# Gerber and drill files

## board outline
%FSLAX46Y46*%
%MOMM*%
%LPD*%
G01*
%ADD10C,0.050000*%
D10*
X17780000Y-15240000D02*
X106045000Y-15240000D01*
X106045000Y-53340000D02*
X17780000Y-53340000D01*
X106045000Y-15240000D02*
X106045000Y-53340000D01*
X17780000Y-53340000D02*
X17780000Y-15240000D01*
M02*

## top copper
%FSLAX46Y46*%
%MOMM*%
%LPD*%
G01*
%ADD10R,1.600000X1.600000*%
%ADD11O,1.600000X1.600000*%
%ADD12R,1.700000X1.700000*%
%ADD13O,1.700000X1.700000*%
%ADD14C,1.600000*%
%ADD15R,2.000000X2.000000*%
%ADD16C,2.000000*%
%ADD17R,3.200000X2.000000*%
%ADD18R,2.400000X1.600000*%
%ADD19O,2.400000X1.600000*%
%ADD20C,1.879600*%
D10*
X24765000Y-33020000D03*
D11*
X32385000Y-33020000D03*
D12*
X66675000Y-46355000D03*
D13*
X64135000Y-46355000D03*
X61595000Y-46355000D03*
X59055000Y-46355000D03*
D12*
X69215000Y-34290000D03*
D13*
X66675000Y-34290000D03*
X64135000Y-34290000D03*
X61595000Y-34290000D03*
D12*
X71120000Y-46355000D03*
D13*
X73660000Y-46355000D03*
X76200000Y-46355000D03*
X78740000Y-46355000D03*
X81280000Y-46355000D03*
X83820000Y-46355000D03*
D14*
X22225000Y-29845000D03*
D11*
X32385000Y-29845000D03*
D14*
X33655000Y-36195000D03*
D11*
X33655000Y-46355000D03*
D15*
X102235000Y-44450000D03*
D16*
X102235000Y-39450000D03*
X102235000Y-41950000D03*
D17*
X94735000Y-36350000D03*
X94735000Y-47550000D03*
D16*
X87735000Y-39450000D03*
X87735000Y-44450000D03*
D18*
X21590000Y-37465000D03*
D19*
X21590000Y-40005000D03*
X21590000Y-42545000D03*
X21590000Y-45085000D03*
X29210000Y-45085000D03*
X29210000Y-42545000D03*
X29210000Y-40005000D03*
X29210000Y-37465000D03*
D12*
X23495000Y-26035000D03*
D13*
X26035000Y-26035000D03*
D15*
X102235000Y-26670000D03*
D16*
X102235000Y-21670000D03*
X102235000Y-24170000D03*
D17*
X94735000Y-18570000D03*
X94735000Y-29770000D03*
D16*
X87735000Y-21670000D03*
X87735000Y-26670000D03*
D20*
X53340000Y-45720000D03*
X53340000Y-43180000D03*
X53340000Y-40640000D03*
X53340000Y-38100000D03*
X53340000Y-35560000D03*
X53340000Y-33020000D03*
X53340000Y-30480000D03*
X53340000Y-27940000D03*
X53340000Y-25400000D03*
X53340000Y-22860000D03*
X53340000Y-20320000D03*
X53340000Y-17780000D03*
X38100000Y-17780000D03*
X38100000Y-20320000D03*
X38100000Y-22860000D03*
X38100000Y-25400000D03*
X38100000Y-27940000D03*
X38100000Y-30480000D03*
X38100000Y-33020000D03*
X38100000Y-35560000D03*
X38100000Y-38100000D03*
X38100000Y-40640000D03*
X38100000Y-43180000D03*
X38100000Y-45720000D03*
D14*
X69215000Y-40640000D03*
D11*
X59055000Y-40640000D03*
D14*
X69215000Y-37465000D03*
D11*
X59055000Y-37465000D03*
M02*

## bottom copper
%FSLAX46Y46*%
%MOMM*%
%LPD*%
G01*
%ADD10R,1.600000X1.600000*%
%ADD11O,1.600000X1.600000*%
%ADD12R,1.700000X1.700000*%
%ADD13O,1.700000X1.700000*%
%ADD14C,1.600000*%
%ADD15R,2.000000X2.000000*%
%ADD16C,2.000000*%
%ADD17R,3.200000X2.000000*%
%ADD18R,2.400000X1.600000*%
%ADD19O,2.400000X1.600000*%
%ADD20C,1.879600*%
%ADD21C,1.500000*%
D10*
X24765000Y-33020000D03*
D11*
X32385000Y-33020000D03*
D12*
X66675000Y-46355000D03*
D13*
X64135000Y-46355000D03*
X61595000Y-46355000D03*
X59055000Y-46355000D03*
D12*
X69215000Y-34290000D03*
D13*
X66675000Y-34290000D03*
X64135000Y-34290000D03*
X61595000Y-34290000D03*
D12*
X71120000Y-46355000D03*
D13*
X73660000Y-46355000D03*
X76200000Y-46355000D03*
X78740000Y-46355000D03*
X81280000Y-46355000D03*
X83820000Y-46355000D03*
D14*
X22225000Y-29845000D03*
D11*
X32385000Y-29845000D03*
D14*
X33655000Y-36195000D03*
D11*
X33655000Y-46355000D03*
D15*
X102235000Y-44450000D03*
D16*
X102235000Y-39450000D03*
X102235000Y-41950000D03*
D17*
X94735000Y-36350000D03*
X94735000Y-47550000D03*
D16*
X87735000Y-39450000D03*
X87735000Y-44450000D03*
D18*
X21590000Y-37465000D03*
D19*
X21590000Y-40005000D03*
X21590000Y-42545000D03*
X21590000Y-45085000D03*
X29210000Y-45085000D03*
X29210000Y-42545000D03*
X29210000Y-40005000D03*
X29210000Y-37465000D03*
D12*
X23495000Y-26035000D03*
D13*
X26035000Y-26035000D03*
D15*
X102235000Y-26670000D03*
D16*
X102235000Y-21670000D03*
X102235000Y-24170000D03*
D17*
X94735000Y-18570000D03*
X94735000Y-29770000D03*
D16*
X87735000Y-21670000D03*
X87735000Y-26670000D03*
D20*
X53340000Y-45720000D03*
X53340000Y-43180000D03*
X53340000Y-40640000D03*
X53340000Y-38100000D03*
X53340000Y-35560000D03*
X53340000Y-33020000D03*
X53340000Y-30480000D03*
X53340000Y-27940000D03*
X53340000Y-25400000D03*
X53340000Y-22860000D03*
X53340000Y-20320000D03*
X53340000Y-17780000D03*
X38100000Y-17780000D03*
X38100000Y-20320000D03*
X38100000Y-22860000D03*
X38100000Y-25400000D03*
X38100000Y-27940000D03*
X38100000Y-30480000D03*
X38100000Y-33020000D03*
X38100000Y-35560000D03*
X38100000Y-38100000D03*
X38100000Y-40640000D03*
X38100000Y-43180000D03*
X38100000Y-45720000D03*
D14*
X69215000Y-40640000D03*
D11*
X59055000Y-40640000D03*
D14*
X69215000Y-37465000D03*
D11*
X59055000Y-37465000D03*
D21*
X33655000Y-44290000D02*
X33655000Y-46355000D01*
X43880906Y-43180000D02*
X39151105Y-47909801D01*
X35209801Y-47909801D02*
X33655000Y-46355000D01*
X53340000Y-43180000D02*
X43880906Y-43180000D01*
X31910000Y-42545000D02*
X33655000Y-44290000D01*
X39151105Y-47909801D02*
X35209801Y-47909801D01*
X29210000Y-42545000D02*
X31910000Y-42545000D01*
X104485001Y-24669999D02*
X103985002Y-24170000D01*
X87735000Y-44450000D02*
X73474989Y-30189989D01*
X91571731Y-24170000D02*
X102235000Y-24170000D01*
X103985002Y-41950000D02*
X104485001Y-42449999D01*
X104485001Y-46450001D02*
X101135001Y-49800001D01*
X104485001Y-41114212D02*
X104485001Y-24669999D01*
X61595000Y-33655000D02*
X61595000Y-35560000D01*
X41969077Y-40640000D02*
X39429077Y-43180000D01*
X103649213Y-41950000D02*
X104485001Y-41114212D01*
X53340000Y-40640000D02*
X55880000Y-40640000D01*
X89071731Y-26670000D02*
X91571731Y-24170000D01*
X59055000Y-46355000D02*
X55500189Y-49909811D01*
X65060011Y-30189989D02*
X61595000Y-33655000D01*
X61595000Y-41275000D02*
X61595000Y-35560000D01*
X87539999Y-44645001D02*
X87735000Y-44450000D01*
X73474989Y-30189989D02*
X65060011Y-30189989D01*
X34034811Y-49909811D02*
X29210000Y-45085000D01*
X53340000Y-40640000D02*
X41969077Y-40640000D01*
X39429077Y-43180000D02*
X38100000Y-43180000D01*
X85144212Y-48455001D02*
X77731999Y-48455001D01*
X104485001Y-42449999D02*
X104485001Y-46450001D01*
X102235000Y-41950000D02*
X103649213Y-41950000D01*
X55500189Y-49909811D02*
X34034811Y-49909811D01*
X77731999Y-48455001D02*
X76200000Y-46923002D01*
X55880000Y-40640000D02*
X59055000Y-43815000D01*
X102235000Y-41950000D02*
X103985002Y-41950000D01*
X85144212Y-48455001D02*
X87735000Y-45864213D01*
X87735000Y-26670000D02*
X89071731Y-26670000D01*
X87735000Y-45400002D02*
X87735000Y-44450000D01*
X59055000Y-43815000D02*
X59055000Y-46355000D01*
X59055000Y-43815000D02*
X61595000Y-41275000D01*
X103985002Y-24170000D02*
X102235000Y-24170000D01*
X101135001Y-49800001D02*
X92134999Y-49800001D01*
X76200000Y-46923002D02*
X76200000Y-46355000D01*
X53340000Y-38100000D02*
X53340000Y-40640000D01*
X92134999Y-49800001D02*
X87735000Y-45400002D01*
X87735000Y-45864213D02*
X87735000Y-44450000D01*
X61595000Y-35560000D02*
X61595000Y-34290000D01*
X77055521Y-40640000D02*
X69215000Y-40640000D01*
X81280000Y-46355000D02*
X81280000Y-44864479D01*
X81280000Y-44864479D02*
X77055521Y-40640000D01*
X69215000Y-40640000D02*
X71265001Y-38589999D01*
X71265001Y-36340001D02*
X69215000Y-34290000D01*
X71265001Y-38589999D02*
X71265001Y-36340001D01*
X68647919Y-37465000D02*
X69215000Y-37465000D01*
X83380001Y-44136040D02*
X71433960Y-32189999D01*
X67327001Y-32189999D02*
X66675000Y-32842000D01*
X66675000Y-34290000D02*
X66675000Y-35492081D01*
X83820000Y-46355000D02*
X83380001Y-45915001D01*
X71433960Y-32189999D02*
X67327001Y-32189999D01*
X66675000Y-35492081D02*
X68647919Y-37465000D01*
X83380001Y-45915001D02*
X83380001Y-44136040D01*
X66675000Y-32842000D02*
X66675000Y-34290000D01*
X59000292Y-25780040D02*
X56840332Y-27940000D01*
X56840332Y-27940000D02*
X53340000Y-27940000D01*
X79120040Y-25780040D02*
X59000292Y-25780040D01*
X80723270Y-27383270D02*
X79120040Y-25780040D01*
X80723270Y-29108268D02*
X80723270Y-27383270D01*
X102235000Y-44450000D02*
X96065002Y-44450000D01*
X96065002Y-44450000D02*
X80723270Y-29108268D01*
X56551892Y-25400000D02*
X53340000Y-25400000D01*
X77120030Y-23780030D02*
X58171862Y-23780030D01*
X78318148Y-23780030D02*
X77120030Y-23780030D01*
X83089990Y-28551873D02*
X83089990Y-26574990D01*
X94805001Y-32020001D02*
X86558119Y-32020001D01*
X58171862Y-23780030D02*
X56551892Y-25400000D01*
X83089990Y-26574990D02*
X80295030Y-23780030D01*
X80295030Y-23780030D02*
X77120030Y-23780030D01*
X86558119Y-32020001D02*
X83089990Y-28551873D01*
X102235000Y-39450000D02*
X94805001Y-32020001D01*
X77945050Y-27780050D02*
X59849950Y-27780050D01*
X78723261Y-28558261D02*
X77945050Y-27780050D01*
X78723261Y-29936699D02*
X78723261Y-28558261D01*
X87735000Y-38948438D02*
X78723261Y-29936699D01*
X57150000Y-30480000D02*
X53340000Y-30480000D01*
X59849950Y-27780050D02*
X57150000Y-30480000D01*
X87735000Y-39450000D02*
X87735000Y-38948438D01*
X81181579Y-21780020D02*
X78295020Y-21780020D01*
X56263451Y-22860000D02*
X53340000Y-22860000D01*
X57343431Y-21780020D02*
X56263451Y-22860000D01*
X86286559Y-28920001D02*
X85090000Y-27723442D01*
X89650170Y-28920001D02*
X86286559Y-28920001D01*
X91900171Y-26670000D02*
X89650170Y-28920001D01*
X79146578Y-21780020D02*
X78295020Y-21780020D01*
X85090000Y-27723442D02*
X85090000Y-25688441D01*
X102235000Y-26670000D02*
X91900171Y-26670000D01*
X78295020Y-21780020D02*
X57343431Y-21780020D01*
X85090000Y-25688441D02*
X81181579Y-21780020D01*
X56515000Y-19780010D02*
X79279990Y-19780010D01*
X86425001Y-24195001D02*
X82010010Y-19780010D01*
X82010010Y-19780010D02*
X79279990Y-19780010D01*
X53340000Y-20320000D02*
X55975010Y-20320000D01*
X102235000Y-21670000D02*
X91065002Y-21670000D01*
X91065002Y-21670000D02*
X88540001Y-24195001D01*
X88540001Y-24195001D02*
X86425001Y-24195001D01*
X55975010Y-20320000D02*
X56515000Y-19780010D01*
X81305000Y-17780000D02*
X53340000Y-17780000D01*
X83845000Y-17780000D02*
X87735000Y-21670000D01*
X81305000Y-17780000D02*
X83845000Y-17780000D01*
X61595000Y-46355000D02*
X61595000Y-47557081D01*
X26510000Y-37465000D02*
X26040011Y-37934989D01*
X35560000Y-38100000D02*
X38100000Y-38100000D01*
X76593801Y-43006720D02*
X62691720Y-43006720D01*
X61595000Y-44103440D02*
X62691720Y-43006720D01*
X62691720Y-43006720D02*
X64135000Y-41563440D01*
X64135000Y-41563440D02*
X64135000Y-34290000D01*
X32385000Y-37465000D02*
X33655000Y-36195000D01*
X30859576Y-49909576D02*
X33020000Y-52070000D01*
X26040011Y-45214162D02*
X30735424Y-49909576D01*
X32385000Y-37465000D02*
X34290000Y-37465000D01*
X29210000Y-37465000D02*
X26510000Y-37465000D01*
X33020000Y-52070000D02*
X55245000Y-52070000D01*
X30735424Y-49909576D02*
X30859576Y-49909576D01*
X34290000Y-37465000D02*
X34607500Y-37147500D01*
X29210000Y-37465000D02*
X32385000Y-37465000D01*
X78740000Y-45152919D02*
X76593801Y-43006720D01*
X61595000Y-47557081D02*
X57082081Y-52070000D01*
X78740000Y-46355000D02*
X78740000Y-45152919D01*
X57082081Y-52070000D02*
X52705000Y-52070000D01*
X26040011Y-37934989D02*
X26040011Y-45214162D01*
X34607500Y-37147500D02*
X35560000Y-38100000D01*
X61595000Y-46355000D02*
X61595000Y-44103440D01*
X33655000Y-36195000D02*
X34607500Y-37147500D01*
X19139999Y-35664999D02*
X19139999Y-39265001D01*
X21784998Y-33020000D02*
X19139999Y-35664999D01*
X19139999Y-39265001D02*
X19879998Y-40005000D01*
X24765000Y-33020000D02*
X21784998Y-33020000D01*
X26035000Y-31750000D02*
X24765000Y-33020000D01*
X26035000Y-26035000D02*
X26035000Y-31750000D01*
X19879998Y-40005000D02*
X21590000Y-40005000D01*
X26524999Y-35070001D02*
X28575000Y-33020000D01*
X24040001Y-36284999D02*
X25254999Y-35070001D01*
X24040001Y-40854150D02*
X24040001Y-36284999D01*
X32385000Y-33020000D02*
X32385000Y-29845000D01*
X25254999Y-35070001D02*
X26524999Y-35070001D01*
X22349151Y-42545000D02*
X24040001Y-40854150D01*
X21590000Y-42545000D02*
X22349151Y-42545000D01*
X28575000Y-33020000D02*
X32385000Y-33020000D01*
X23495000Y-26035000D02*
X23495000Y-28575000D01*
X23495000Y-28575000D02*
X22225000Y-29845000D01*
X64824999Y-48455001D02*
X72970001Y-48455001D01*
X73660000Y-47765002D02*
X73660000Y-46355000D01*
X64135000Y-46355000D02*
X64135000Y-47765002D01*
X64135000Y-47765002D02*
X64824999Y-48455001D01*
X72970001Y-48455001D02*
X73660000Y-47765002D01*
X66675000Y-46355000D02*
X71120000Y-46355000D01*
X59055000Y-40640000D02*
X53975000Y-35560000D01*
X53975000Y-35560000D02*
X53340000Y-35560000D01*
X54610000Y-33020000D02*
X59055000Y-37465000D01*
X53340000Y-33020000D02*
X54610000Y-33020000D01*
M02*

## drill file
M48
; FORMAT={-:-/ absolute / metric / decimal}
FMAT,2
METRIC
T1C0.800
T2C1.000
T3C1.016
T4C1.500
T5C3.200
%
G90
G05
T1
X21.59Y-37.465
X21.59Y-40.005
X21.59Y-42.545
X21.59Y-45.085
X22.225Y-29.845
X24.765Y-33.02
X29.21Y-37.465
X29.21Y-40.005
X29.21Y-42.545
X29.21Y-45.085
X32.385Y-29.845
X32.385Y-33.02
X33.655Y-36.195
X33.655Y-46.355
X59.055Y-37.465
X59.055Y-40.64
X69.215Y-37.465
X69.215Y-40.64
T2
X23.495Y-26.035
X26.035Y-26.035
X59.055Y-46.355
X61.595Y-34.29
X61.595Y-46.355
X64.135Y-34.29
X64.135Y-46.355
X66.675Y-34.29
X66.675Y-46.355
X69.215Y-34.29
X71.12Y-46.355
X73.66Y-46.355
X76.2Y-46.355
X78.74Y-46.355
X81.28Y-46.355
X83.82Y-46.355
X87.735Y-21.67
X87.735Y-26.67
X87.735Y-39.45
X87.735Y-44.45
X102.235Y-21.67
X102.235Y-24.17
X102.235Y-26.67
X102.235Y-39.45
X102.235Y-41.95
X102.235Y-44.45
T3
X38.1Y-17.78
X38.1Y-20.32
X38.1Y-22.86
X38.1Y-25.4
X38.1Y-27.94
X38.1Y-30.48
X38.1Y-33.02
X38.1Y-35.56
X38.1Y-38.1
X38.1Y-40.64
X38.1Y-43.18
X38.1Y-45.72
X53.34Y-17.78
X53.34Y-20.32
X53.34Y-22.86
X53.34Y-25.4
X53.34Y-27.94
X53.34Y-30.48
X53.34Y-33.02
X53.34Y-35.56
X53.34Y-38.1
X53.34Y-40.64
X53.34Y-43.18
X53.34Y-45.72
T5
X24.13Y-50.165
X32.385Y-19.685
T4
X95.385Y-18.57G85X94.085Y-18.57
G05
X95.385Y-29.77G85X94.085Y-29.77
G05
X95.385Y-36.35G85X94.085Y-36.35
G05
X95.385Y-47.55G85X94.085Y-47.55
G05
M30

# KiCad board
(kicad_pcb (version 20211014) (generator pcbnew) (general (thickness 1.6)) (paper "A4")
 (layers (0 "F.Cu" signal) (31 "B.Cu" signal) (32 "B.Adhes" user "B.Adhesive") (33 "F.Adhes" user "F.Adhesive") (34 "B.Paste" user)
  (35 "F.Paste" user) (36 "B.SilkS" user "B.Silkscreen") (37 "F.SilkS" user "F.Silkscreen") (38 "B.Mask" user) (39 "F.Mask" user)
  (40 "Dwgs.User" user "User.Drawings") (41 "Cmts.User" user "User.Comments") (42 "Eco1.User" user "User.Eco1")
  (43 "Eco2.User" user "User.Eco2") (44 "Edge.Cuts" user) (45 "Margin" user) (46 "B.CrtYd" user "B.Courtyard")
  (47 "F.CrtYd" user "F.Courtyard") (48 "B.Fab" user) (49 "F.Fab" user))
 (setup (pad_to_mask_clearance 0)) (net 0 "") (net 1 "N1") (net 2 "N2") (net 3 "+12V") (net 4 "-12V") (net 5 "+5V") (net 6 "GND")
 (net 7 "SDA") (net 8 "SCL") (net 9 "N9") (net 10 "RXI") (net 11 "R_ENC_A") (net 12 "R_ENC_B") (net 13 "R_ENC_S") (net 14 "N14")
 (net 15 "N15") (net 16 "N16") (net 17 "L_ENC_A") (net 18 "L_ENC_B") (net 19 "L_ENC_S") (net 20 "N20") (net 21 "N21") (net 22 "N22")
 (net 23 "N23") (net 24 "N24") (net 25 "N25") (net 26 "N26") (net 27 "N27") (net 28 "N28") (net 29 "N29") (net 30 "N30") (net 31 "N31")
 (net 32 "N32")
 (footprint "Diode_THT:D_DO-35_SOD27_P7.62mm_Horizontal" (layer "F.Cu") (at 24.765 33.02)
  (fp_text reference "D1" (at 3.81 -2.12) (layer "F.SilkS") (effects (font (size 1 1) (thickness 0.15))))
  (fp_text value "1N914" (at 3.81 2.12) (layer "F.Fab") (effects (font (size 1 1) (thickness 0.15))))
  (pad "1" thru_hole rect locked (at 0 0) (size 1.6 1.6) (drill 0.8) (layers *.Cu *.Mask) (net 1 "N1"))
  (pad "2" thru_hole oval locked (at 7.62 0) (size 1.6 1.6) (drill 0.8) (layers *.Cu *.Mask) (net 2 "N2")))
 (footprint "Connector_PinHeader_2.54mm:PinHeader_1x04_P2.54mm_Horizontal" (layer "F.Cu") (at 66.675 46.355 -90)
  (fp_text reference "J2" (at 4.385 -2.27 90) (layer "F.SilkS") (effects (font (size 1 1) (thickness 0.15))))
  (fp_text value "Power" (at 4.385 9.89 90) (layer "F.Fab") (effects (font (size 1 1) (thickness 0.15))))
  (pad "1" thru_hole rect locked (at 0 0 270) (size 1.7 1.7) (drill 1) (layers *.Cu *.Mask) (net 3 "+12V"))
  (pad "2" thru_hole oval locked (at 0 2.54 270) (size 1.7 1.7) (drill 1) (layers *.Cu *.Mask) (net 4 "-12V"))
  (pad "3" thru_hole oval locked (at 0 5.08 270) (size 1.7 1.7) (drill 1) (layers *.Cu *.Mask) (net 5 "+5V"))
  (pad "4" thru_hole oval locked (at 0 7.62 270) (size 1.7 1.7) (drill 1) (layers *.Cu *.Mask) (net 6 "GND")))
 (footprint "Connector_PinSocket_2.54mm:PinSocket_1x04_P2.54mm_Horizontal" (layer "F.Cu") (at 69.215 34.29 -90)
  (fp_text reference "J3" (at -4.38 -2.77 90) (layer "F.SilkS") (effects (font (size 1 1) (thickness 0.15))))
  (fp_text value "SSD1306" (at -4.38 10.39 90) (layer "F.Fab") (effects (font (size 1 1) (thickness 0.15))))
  (pad "1" thru_hole rect locked (at 0 0 270) (size 1.7 1.7) (drill 1) (layers *.Cu *.Mask) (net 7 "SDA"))
  (pad "2" thru_hole oval locked (at 0 2.54 270) (size 1.7 1.7) (drill 1) (layers *.Cu *.Mask) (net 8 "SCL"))
  (pad "3" thru_hole oval locked (at 0 5.08 270) (size 1.7 1.7) (drill 1) (layers *.Cu *.Mask) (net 5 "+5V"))
  (pad "4" thru_hole oval locked (at 0 7.62 270) (size 1.7 1.7) (drill 1) (layers *.Cu *.Mask) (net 6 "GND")))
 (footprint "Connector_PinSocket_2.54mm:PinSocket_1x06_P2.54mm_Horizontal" (layer "F.Cu") (at 71.12 46.355 90)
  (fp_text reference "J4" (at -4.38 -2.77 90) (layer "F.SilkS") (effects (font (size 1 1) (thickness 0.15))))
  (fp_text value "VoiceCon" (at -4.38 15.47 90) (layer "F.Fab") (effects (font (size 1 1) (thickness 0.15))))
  (pad "1" thru_hole rect locked (at 0 0 90) (size 1.7 1.7) (drill 1) (layers *.Cu *.Mask) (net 3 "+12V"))
  (pad "2" thru_hole oval locked (at 0 2.54 90) (size 1.7 1.7) (drill 1) (layers *.Cu *.Mask) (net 4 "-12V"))
  (pad "3" thru_hole oval locked (at 0 5.08 90) (size 1.7 1.7) (drill 1) (layers *.Cu *.Mask) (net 6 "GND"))
  (pad "4" thru_hole oval locked (at 0 7.62 90) (size 1.7 1.7) (drill 1) (layers *.Cu *.Mask) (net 5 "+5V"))
  (pad "5" thru_hole oval locked (at 0 10.16 90) (size 1.7 1.7) (drill 1) (layers *.Cu *.Mask) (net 7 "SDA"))
  (pad "6" thru_hole oval locked (at 0 12.7 90) (size 1.7 1.7) (drill 1) (layers *.Cu *.Mask) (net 8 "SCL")))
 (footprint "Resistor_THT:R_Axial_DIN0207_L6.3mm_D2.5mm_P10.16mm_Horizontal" (layer "F.Cu") (at 22.225 29.845)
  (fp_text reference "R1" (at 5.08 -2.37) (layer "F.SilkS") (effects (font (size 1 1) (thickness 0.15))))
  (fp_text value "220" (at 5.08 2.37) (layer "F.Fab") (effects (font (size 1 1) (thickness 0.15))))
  (pad "1" thru_hole circle locked (at 0 0) (size 1.6 1.6) (drill 0.8) (layers *.Cu *.Mask) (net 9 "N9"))
  (pad "2" thru_hole oval locked (at 10.16 0) (size 1.6 1.6) (drill 0.8) (layers *.Cu *.Mask) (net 2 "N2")))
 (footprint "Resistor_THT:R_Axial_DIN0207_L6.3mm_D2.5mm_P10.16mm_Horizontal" (layer "F.Cu") (at 33.655 36.195 -90)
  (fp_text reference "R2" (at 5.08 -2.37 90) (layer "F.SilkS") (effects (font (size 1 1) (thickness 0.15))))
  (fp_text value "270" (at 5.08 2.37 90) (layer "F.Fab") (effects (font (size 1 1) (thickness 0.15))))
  (pad "1" thru_hole circle locked (at 0 0 270) (size 1.6 1.6) (drill 0.8) (layers *.Cu *.Mask) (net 5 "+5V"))
  (pad "2" thru_hole oval locked (at 10.16 0 270) (size 1.6 1.6) (drill 0.8) (layers *.Cu *.Mask) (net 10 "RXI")))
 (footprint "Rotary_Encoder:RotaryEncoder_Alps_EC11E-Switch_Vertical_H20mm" (layer "F.Cu") (at 102.235 44.45 180)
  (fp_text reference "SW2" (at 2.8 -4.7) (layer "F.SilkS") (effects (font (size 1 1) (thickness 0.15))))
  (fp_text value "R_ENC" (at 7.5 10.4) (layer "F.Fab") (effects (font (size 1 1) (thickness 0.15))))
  (pad "A" thru_hole rect locked (at 0 0 180) (size 2 2) (drill 1) (layers *.Cu *.Mask) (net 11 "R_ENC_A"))
  (pad "B" thru_hole circle locked (at 0 5 180) (size 2 2) (drill 1) (layers *.Cu *.Mask) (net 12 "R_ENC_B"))
  (pad "C" thru_hole circle locked (at 0 2.5 180) (size 2 2) (drill 1) (layers *.Cu *.Mask) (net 6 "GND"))
  (pad "MP" thru_hole rect locked (at 7.5 8.1 180) (size 3.2 2) (drill oval 2.8 1.5) (layers *.Cu *.Mask))
  (pad "MP" thru_hole rect locked (at 7.5 -3.1 180) (size 3.2 2) (drill oval 2.8 1.5) (layers *.Cu *.Mask))
  (pad "S1" thru_hole circle locked (at 14.5 5 180) (size 2 2) (drill 1) (layers *.Cu *.Mask) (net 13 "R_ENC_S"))
  (pad "S2" thru_hole circle locked (at 14.5 0 180) (size 2 2) (drill 1) (layers *.Cu *.Mask) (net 6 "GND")))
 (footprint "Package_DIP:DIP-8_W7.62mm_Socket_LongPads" (layer "F.Cu") (at 21.59 37.465)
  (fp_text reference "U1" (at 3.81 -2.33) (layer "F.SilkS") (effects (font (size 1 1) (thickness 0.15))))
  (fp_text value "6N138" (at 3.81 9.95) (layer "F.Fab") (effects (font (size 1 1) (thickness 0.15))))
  (pad "1" thru_hole rect locked (at 0 0) (size 2.4 1.6) (drill 0.8) (layers *.Cu *.Mask) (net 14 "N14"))
  (pad "2" thru_hole oval locked (at 0 2.54) (size 2.4 1.6) (drill 0.8) (layers *.Cu *.Mask) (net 1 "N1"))
  (pad "3" thru_hole oval locked (at 0 5.08) (size 2.4 1.6) (drill 0.8) (layers *.Cu *.Mask) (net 2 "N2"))
  (pad "4" thru_hole oval locked (at 0 7.62) (size 2.4 1.6) (drill 0.8) (layers *.Cu *.Mask) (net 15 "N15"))
  (pad "5" thru_hole oval locked (at 7.62 7.62) (size 2.4 1.6) (drill 0.8) (layers *.Cu *.Mask) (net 6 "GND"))
  (pad "6" thru_hole oval locked (at 7.62 5.08) (size 2.4 1.6) (drill 0.8) (layers *.Cu *.Mask) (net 10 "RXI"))
  (pad "7" thru_hole oval locked (at 7.62 2.54) (size 2.4 1.6) (drill 0.8) (layers *.Cu *.Mask) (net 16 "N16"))
  (pad "8" thru_hole oval locked (at 7.62 0) (size 2.4 1.6) (drill 0.8) (layers *.Cu *.Mask) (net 5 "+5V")))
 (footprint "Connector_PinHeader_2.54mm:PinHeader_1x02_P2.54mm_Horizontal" (layer "F.Cu") (at 23.495 26.035 90)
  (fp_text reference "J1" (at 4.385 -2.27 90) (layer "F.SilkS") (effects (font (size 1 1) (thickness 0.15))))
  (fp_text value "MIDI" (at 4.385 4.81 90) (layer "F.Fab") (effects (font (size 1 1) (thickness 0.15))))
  (pad "1" thru_hole rect locked (at 0 0 90) (size 1.7 1.7) (drill 1) (layers *.Cu *.Mask) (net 9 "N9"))
  (pad "2" thru_hole oval locked (at 0 2.54 90) (size 1.7 1.7) (drill 1) (layers *.Cu *.Mask) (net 1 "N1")))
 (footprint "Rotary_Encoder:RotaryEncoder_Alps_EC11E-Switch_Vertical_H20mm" (layer "F.Cu") (at 102.235 26.67 180)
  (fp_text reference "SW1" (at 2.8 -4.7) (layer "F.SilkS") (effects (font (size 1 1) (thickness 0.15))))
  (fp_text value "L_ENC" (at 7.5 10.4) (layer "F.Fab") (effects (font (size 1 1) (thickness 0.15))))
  (pad "A" thru_hole rect locked (at 0 0 180) (size 2 2) (drill 1) (layers *.Cu *.Mask) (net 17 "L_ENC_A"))
  (pad "B" thru_hole circle locked (at 0 5 180) (size 2 2) (drill 1) (layers *.Cu *.Mask) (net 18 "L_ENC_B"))
  (pad "C" thru_hole circle locked (at 0 2.5 180) (size 2 2) (drill 1) (layers *.Cu *.Mask) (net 6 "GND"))
  (pad "MP" thru_hole rect locked (at 7.5 8.1 180) (size 3.2 2) (drill oval 2.8 1.5) (layers *.Cu *.Mask))
  (pad "MP" thru_hole rect locked (at 7.5 -3.1 180) (size 3.2 2) (drill oval 2.8 1.5) (layers *.Cu *.Mask))
  (pad "S1" thru_hole circle locked (at 14.5 5 180) (size 2 2) (drill 1) (layers *.Cu *.Mask) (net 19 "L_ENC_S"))
  (pad "S2" thru_hole circle locked (at 14.5 0 180) (size 2 2) (drill 1) (layers *.Cu *.Mask) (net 6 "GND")))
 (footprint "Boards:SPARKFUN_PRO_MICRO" (layer "F.Cu") (at 45.72 33.02 180)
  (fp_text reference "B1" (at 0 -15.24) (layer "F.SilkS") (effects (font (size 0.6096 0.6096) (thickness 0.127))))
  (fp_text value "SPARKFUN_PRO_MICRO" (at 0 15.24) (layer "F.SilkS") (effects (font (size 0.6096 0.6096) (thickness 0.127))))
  (pad "1" thru_hole circle locked (at -7.62 -12.7 180) (size 1.8796 1.8796) (drill 1.016) (layers *.Cu *.Mask) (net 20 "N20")
   (solder_mask_margin 0.1016))
  (pad "2" thru_hole circle locked (at -7.62 -10.16 180) (size 1.8796 1.8796) (drill 1.016) (layers *.Cu *.Mask) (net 10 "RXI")
   (solder_mask_margin 0.1016))
  (pad "3" thru_hole circle locked (at -7.62 -7.62 180) (size 1.8796 1.8796) (drill 1.016) (layers *.Cu *.Mask) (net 6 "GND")
   (solder_mask_margin 0.1016))
  (pad "4" thru_hole circle locked (at -7.62 -5.08 180) (size 1.8796 1.8796) (drill 1.016) (layers *.Cu *.Mask) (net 6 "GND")
   (solder_mask_margin 0.1016))
  (pad "5" thru_hole circle locked (at -7.62 -2.54 180) (size 1.8796 1.8796) (drill 1.016) (layers *.Cu *.Mask) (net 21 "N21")
   (solder_mask_margin 0.1016))
  (pad "6" thru_hole circle locked (at -7.62 0 180) (size 1.8796 1.8796) (drill 1.016) (layers *.Cu *.Mask) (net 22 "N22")
   (solder_mask_margin 0.1016))
  (pad "7" thru_hole circle locked (at -7.62 2.54 180) (size 1.8796 1.8796) (drill 1.016) (layers *.Cu *.Mask) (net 13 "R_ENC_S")
   (solder_mask_margin 0.1016))
  (pad "8" thru_hole circle locked (at -7.62 5.08 180) (size 1.8796 1.8796) (drill 1.016) (layers *.Cu *.Mask) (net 11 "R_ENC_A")
   (solder_mask_margin 0.1016))
  (pad "9" thru_hole circle locked (at -7.62 7.62 180) (size 1.8796 1.8796) (drill 1.016) (layers *.Cu *.Mask) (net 12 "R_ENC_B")
   (solder_mask_margin 0.1016))
  (pad "10" thru_hole circle locked (at -7.62 10.16 180) (size 1.8796 1.8796) (drill 1.016) (layers *.Cu *.Mask) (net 17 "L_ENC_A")
   (solder_mask_margin 0.1016))
  (pad "11" thru_hole circle locked (at -7.62 12.7 180) (size 1.8796 1.8796) (drill 1.016) (layers *.Cu *.Mask) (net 18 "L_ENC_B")
   (solder_mask_margin 0.1016))
  (pad "12" thru_hole circle locked (at -7.62 15.24 180) (size 1.8796 1.8796) (drill 1.016) (layers *.Cu *.Mask) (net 19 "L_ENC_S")
   (solder_mask_margin 0.1016))
  (pad "13" thru_hole circle locked (at 7.62 15.24 180) (size 1.8796 1.8796) (drill 1.016) (layers *.Cu *.Mask) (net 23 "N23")
   (solder_mask_margin 0.1016))
  (pad "14" thru_hole circle locked (at 7.62 12.7 180) (size 1.8796 1.8796) (drill 1.016) (layers *.Cu *.Mask) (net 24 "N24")
   (solder_mask_margin 0.1016))
  (pad "15" thru_hole circle locked (at 7.62 10.16 180) (size 1.8796 1.8796) (drill 1.016) (layers *.Cu *.Mask) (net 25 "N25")
   (solder_mask_margin 0.1016))
  (pad "16" thru_hole circle locked (at 7.62 7.62 180) (size 1.8796 1.8796) (drill 1.016) (layers *.Cu *.Mask) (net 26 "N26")
   (solder_mask_margin 0.1016))
  (pad "17" thru_hole circle locked (at 7.62 5.08 180) (size 1.8796 1.8796) (drill 1.016) (layers *.Cu *.Mask) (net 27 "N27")
   (solder_mask_margin 0.1016))
  (pad "18" thru_hole circle locked (at 7.62 2.54 180) (size 1.8796 1.8796) (drill 1.016) (layers *.Cu *.Mask) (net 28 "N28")
   (solder_mask_margin 0.1016))
  (pad "19" thru_hole circle locked (at 7.62 0 180) (size 1.8796 1.8796) (drill 1.016) (layers *.Cu *.Mask) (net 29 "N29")
   (solder_mask_margin 0.1016))
  (pad "20" thru_hole circle locked (at 7.62 -2.54 180) (size 1.8796 1.8796) (drill 1.016) (layers *.Cu *.Mask) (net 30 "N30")
   (solder_mask_margin 0.1016))
  (pad "21" thru_hole circle locked (at 7.62 -5.08 180) (size 1.8796 1.8796) (drill 1.016) (layers *.Cu *.Mask) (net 5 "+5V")
   (solder_mask_margin 0.1016))
  (pad "22" thru_hole circle locked (at 7.62 -7.62 180) (size 1.8796 1.8796) (drill 1.016) (layers *.Cu *.Mask) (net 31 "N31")
   (solder_mask_margin 0.1016))
  (pad "23" thru_hole circle locked (at 7.62 -10.16 180) (size 1.8796 1.8796) (drill 1.016) (layers *.Cu *.Mask) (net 6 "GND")
   (solder_mask_margin 0.1016))
  (pad "24" thru_hole circle locked (at 7.62 -12.7 180) (size 1.8796 1.8796) (drill 1.016) (layers *.Cu *.Mask) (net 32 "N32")
   (solder_mask_margin 0.1016)))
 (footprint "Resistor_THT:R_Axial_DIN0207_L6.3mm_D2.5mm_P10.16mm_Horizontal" (layer "F.Cu") (at 69.215 40.64 180)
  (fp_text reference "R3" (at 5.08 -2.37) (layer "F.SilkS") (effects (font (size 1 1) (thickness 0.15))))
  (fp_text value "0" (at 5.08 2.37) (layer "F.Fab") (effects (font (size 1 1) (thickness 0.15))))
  (pad "1" thru_hole circle locked (at 0 0 180) (size 1.6 1.6) (drill 0.8) (layers *.Cu *.Mask) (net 7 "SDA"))
  (pad "2" thru_hole oval locked (at 10.16 0 180) (size 1.6 1.6) (drill 0.8) (layers *.Cu *.Mask) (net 21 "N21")))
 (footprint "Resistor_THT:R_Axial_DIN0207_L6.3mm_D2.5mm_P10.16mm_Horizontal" (layer "F.Cu") (at 69.215 37.465 180)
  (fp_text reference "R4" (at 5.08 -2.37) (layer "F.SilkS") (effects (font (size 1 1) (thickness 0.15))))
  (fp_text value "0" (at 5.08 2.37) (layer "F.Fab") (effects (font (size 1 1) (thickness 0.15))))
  (pad "1" thru_hole circle locked (at 0 0 180) (size 1.6 1.6) (drill 0.8) (layers *.Cu *.Mask) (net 8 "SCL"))
  (pad "2" thru_hole oval locked (at 10.16 0 180) (size 1.6 1.6) (drill 0.8) (layers *.Cu *.Mask) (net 22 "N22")))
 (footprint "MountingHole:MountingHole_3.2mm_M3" (layer "F.Cu") (at 32.385 19.685)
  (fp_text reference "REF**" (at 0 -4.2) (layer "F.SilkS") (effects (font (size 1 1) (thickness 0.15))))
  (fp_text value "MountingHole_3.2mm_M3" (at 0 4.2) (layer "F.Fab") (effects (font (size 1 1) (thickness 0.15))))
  (pad "" np_thru_hole circle locked (at 0 0) (size 3.2 3.2) (drill 3.2) (layers *.Cu *.Mask)))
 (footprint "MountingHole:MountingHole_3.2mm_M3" (layer "F.Cu") (at 24.13 50.165)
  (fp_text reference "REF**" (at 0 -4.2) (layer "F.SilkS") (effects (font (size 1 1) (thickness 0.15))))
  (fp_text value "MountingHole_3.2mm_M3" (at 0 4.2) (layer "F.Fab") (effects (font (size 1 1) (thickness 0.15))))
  (pad "" np_thru_hole circle locked (at 0 0) (size 3.2 3.2) (drill 3.2) (layers *.Cu *.Mask)))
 (gr_line (start 17.78 15.24) (end 106.045 15.24) (layer "Edge.Cuts") (width 0.05))
 (gr_line (start 106.045 53.34) (end 17.78 53.34) (layer "Edge.Cuts") (width 0.05))
 (gr_line (start 106.045 15.24) (end 106.045 53.34) (layer "Edge.Cuts") (width 0.05))
 (gr_line (start 17.78 53.34) (end 17.78 15.24) (layer "Edge.Cuts") (width 0.05))
 (segment (start 33.655 44.29) (end 33.655 46.355) (width 1.5) (layer "B.Cu") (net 10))
 (segment (start 43.880906 43.18) (end 39.151105 47.909801) (width 1.5) (layer "B.Cu") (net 10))
 (segment (start 35.209801 47.909801) (end 33.655 46.355) (width 1.5) (layer "B.Cu") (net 10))
 (segment (start 53.34 43.18) (end 43.880906 43.18) (width 1.5) (layer "B.Cu") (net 10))
 (segment (start 31.91 42.545) (end 33.655 44.29) (width 1.5) (layer "B.Cu") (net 10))
 (segment (start 39.151105 47.909801) (end 35.209801 47.909801) (width 1.5) (layer "B.Cu") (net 10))
 (segment (start 29.21 42.545) (end 31.91 42.545) (width 1.5) (layer "B.Cu") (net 10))
 (segment (start 104.485001 24.669999) (end 103.985002 24.17) (width 1.5) (layer "B.Cu") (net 6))
 (segment (start 87.735 44.45) (end 73.474989 30.189989) (width 1.5) (layer "B.Cu") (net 6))
 (segment (start 91.571731 24.17) (end 102.235 24.17) (width 1.5) (layer "B.Cu") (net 6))
 (segment (start 103.985002 41.95) (end 104.485001 42.449999) (width 1.5) (layer "B.Cu") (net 6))
 (segment (start 104.485001 46.450001) (end 101.135001 49.800001) (width 1.5) (layer "B.Cu") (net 6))
 (segment (start 104.485001 41.114212) (end 104.485001 24.669999) (width 1.5) (layer "B.Cu") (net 6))
 (segment (start 61.595 33.655) (end 61.595 35.56) (width 1.5) (layer "B.Cu") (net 6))
 (segment (start 41.969077 40.64) (end 39.429077 43.18) (width 1.5) (layer "B.Cu") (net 6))
 (segment (start 103.649213 41.95) (end 104.485001 41.114212) (width 1.5) (layer "B.Cu") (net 6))
 (segment (start 53.34 40.64) (end 55.88 40.64) (width 1.5) (layer "B.Cu") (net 6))
 (segment (start 89.071731 26.67) (end 91.571731 24.17) (width 1.5) (layer "B.Cu") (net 6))
 (segment (start 59.055 46.355) (end 55.500189 49.909811) (width 1.5) (layer "B.Cu") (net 6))
 (segment (start 65.060011 30.189989) (end 61.595 33.655) (width 1.5) (layer "B.Cu") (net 6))
 (segment (start 61.595 41.275) (end 61.595 35.56) (width 1.5) (layer "B.Cu") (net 6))
 (segment (start 87.539999 44.645001) (end 87.735 44.45) (width 1.5) (layer "B.Cu") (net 6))
 (segment (start 73.474989 30.189989) (end 65.060011 30.189989) (width 1.5) (layer "B.Cu") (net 6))
 (segment (start 34.034811 49.909811) (end 29.21 45.085) (width 1.5) (layer "B.Cu") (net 6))
 (segment (start 53.34 40.64) (end 41.969077 40.64) (width 1.5) (layer "B.Cu") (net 6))
 (segment (start 39.429077 43.18) (end 38.1 43.18) (width 1.5) (layer "B.Cu") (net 6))
 (segment (start 85.144212 48.455001) (end 77.731999 48.455001) (width 1.5) (layer "B.Cu") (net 6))
 (segment (start 104.485001 42.449999) (end 104.485001 46.450001) (width 1.5) (layer "B.Cu") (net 6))
 (segment (start 102.235 41.95) (end 103.649213 41.95) (width 1.5) (layer "B.Cu") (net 6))
 (segment (start 55.500189 49.909811) (end 34.034811 49.909811) (width 1.5) (layer "B.Cu") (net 6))
 (segment (start 77.731999 48.455001) (end 76.2 46.923002) (width 1.5) (layer "B.Cu") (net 6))
 (segment (start 55.88 40.64) (end 59.055 43.815) (width 1.5) (layer "B.Cu") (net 6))
 (segment (start 102.235 41.95) (end 103.985002 41.95) (width 1.5) (layer "B.Cu") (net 6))
 (segment (start 85.144212 48.455001) (end 87.735 45.864213) (width 1.5) (layer "B.Cu") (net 6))
 (segment (start 87.735 26.67) (end 89.071731 26.67) (width 1.5) (layer "B.Cu") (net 6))
 (segment (start 87.735 45.400002) (end 87.735 44.45) (width 1.5) (layer "B.Cu") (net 6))
 (segment (start 59.055 43.815) (end 59.055 46.355) (width 1.5) (layer "B.Cu") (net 6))
 (segment (start 59.055 43.815) (end 61.595 41.275) (width 1.5) (layer "B.Cu") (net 6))
 (segment (start 103.985002 24.17) (end 102.235 24.17) (width 1.5) (layer "B.Cu") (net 6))
 (segment (start 101.135001 49.800001) (end 92.134999 49.800001) (width 1.5) (layer "B.Cu") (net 6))
 (segment (start 76.2 46.923002) (end 76.2 46.355) (width 1.5) (layer "B.Cu") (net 6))
 (segment (start 53.34 38.1) (end 53.34 40.64) (width 1.5) (layer "B.Cu") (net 6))
 (segment (start 92.134999 49.800001) (end 87.735 45.400002) (width 1.5) (layer "B.Cu") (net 6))
 (segment (start 87.735 45.864213) (end 87.735 44.45) (width 1.5) (layer "B.Cu") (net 6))
 (segment (start 61.595 35.56) (end 61.595 34.29) (width 1.5) (layer "B.Cu") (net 6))
 (segment (start 77.055521 40.64) (end 69.215 40.64) (width 1.5) (layer "B.Cu") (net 7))
 (segment (start 81.28 46.355) (end 81.28 44.864479) (width 1.5) (layer "B.Cu") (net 7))
 (segment (start 81.28 44.864479) (end 77.055521 40.64) (width 1.5) (layer "B.Cu") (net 7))
 (segment (start 69.215 40.64) (end 71.265001 38.589999) (width 1.5) (layer "B.Cu") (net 7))
 (segment (start 71.265001 36.340001) (end 69.215 34.29) (width 1.5) (layer "B.Cu") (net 7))
 (segment (start 71.265001 38.589999) (end 71.265001 36.340001) (width 1.5) (layer "B.Cu") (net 7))
 (segment (start 68.647919 37.465) (end 69.215 37.465) (width 1.5) (layer "B.Cu") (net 8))
 (segment (start 83.380001 44.13604) (end 71.43396 32.189999) (width 1.5) (layer "B.Cu") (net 8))
 (segment (start 67.327001 32.189999) (end 66.675 32.842) (width 1.5) (layer "B.Cu") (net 8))
 (segment (start 66.675 34.29) (end 66.675 35.492081) (width 1.5) (layer "B.Cu") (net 8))
 (segment (start 83.82 46.355) (end 83.380001 45.915001) (width 1.5) (layer "B.Cu") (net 8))
 (segment (start 71.43396 32.189999) (end 67.327001 32.189999) (width 1.5) (layer "B.Cu") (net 8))
 (segment (start 66.675 35.492081) (end 68.647919 37.465) (width 1.5) (layer "B.Cu") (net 8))
 (segment (start 83.380001 45.915001) (end 83.380001 44.13604) (width 1.5) (layer "B.Cu") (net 8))
 (segment (start 66.675 32.842) (end 66.675 34.29) (width 1.5) (layer "B.Cu") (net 8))
 (segment (start 59.000292 25.78004) (end 56.840332 27.94) (width 1.5) (layer "B.Cu") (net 11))
 (segment (start 56.840332 27.94) (end 53.34 27.94) (width 1.5) (layer "B.Cu") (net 11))
 (segment (start 79.12004 25.78004) (end 59.000292 25.78004) (width 1.5) (layer "B.Cu") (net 11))
 (segment (start 80.72327 27.38327) (end 79.12004 25.78004) (width 1.5) (layer "B.Cu") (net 11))
 (segment (start 80.72327 29.108268) (end 80.72327 27.38327) (width 1.5) (layer "B.Cu") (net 11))
 (segment (start 102.235 44.45) (end 96.065002 44.45) (width 1.5) (layer "B.Cu") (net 11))
 (segment (start 96.065002 44.45) (end 80.72327 29.108268) (width 1.5) (layer "B.Cu") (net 11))
 (segment (start 56.551892 25.4) (end 53.34 25.4) (width 1.5) (layer "B.Cu") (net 12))
 (segment (start 77.12003 23.78003) (end 58.171862 23.78003) (width 1.5) (layer "B.Cu") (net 12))
 (segment (start 78.318148 23.78003) (end 77.12003 23.78003) (width 1.5) (layer "B.Cu") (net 12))
 (segment (start 83.08999 28.551873) (end 83.08999 26.57499) (width 1.5) (layer "B.Cu") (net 12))
 (segment (start 94.805001 32.020001) (end 86.558119 32.020001) (width 1.5) (layer "B.Cu") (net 12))
 (segment (start 58.171862 23.78003) (end 56.551892 25.4) (width 1.5) (layer "B.Cu") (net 12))
 (segment (start 83.08999 26.57499) (end 80.29503 23.78003) (width 1.5) (layer "B.Cu") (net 12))
 (segment (start 80.29503 23.78003) (end 77.12003 23.78003) (width 1.5) (layer "B.Cu") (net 12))
 (segment (start 86.558119 32.020001) (end 83.08999 28.551873) (width 1.5) (layer "B.Cu") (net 12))
 (segment (start 102.235 39.45) (end 94.805001 32.020001) (width 1.5) (layer "B.Cu") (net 12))
 (segment (start 77.94505 27.78005) (end 59.84995 27.78005) (width 1.5) (layer "B.Cu") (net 13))
 (segment (start 78.723261 28.558261) (end 77.94505 27.78005) (width 1.5) (layer "B.Cu") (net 13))
 (segment (start 78.723261 29.936699) (end 78.723261 28.558261) (width 1.5) (layer "B.Cu") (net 13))
 (segment (start 87.735 38.948438) (end 78.723261 29.936699) (width 1.5) (layer "B.Cu") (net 13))
 (segment (start 57.15 30.48) (end 53.34 30.48) (width 1.5) (layer "B.Cu") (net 13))
 (segment (start 59.84995 27.78005) (end 57.15 30.48) (width 1.5) (layer "B.Cu") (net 13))
 (segment (start 87.735 39.45) (end 87.735 38.948438) (width 1.5) (layer "B.Cu") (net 13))
 (segment (start 81.181579 21.78002) (end 78.29502 21.78002) (width 1.5) (layer "B.Cu") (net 17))
 (segment (start 56.263451 22.86) (end 53.34 22.86) (width 1.5) (layer "B.Cu") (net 17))
 (segment (start 57.343431 21.78002) (end 56.263451 22.86) (width 1.5) (layer "B.Cu") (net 17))
 (segment (start 86.286559 28.920001) (end 85.09 27.723442) (width 1.5) (layer "B.Cu") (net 17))
 (segment (start 89.65017 28.920001) (end 86.286559 28.920001) (width 1.5) (layer "B.Cu") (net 17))
 (segment (start 91.900171 26.67) (end 89.65017 28.920001) (width 1.5) (layer "B.Cu") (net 17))
 (segment (start 79.146578 21.78002) (end 78.29502 21.78002) (width 1.5) (layer "B.Cu") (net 17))
 (segment (start 85.09 27.723442) (end 85.09 25.688441) (width 1.5) (layer "B.Cu") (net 17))
 (segment (start 102.235 26.67) (end 91.900171 26.67) (width 1.5) (layer "B.Cu") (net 17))
 (segment (start 78.29502 21.78002) (end 57.343431 21.78002) (width 1.5) (layer "B.Cu") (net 17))
 (segment (start 85.09 25.688441) (end 81.181579 21.78002) (width 1.5) (layer "B.Cu") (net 17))
 (segment (start 56.515 19.78001) (end 79.27999 19.78001) (width 1.5) (layer "B.Cu") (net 18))
 (segment (start 86.425001 24.195001) (end 82.01001 19.78001) (width 1.5) (layer "B.Cu") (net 18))
 (segment (start 82.01001 19.78001) (end 79.27999 19.78001) (width 1.5) (layer "B.Cu") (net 18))
 (segment (start 53.34 20.32) (end 55.97501 20.32) (width 1.5) (layer "B.Cu") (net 18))
 (segment (start 102.235 21.67) (end 91.065002 21.67) (width 1.5) (layer "B.Cu") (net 18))
 (segment (start 91.065002 21.67) (end 88.540001 24.195001) (width 1.5) (layer "B.Cu") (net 18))
 (segment (start 88.540001 24.195001) (end 86.425001 24.195001) (width 1.5) (layer "B.Cu") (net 18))
 (segment (start 55.97501 20.32) (end 56.515 19.78001) (width 1.5) (layer "B.Cu") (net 18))
 (segment (start 81.305 17.78) (end 53.34 17.78) (width 1.5) (layer "B.Cu") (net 19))
 (segment (start 83.845 17.78) (end 87.735 21.67) (width 1.5) (layer "B.Cu") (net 19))
 (segment (start 81.305 17.78) (end 83.845 17.78) (width 1.5) (layer "B.Cu") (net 19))
 (segment (start 61.595 46.355) (end 61.595 47.557081) (width 1.5) (layer "B.Cu") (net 5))
 (segment (start 26.51 37.465) (end 26.040011 37.934989) (width 1.5) (layer "B.Cu") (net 5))
 (segment (start 35.56 38.1) (end 38.1 38.1) (width 1.5) (layer "B.Cu") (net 5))
 (segment (start 76.593801 43.00672) (end 62.69172 43.00672) (width 1.5) (layer "B.Cu") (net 5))
 (segment (start 61.595 44.10344) (end 62.69172 43.00672) (width 1.5) (layer "B.Cu") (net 5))
 (segment (start 62.69172 43.00672) (end 64.135 41.56344) (width 1.5) (layer "B.Cu") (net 5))
 (segment (start 64.135 41.56344) (end 64.135 34.29) (width 1.5) (layer "B.Cu") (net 5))
 (segment (start 32.385 37.465) (end 33.655 36.195) (width 1.5) (layer "B.Cu") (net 5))
 (segment (start 30.859576 49.909576) (end 33.02 52.07) (width 1.5) (layer "B.Cu") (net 5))
 (segment (start 26.040011 45.214162) (end 30.735424 49.909576) (width 1.5) (layer "B.Cu") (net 5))
 (segment (start 32.385 37.465) (end 34.29 37.465) (width 1.5) (layer "B.Cu") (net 5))
 (segment (start 29.21 37.465) (end 26.51 37.465) (width 1.5) (layer "B.Cu") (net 5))
 (segment (start 33.02 52.07) (end 55.245 52.07) (width 1.5) (layer "B.Cu") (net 5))
 (segment (start 30.735424 49.909576) (end 30.859576 49.909576) (width 1.5) (layer "B.Cu") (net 5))
 (segment (start 34.29 37.465) (end 34.6075 37.1475) (width 1.5) (layer "B.Cu") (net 5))
 (segment (start 29.21 37.465) (end 32.385 37.465) (width 1.5) (layer "B.Cu") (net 5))
 (segment (start 78.74 45.152919) (end 76.593801 43.00672) (width 1.5) (layer "B.Cu") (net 5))
 (segment (start 61.595 47.557081) (end 57.082081 52.07) (width 1.5) (layer "B.Cu") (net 5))
 (segment (start 78.74 46.355) (end 78.74 45.152919) (width 1.5) (layer "B.Cu") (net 5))
 (segment (start 57.082081 52.07) (end 52.705 52.07) (width 1.5) (layer "B.Cu") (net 5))
 (segment (start 26.040011 37.934989) (end 26.040011 45.214162) (width 1.5) (layer "B.Cu") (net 5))
 (segment (start 34.6075 37.1475) (end 35.56 38.1) (width 1.5) (layer "B.Cu") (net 5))
 (segment (start 61.595 46.355) (end 61.595 44.10344) (width 1.5) (layer "B.Cu") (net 5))
 (segment (start 33.655 36.195) (end 34.6075 37.1475) (width 1.5) (layer "B.Cu") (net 5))
 (segment (start 19.139999 35.664999) (end 19.139999 39.265001) (width 1.5) (layer "B.Cu") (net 1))
 (segment (start 21.784998 33.02) (end 19.139999 35.664999) (width 1.5) (layer "B.Cu") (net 1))
 (segment (start 19.139999 39.265001) (end 19.879998 40.005) (width 1.5) (layer "B.Cu") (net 1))
 (segment (start 24.765 33.02) (end 21.784998 33.02) (width 1.5) (layer "B.Cu") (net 1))
 (segment (start 26.035 31.75) (end 24.765 33.02) (width 1.5) (layer "B.Cu") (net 1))
 (segment (start 26.035 26.035) (end 26.035 31.75) (width 1.5) (layer "B.Cu") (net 1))
 (segment (start 19.879998 40.005) (end 21.59 40.005) (width 1.5) (layer "B.Cu") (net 1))
 (segment (start 26.524999 35.070001) (end 28.575 33.02) (width 1.5) (layer "B.Cu") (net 2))
 (segment (start 24.040001 36.284999) (end 25.254999 35.070001) (width 1.5) (layer "B.Cu") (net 2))
 (segment (start 24.040001 40.85415) (end 24.040001 36.284999) (width 1.5) (layer "B.Cu") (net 2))
 (segment (start 32.385 33.02) (end 32.385 29.845) (width 1.5) (layer "B.Cu") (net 2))
 (segment (start 25.254999 35.070001) (end 26.524999 35.070001) (width 1.5) (layer "B.Cu") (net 2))
 (segment (start 22.349151 42.545) (end 24.040001 40.85415) (width 1.5) (layer "B.Cu") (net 2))
 (segment (start 21.59 42.545) (end 22.349151 42.545) (width 1.5) (layer "B.Cu") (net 2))
 (segment (start 28.575 33.02) (end 32.385 33.02) (width 1.5) (layer "B.Cu") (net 2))
 (segment (start 23.495 26.035) (end 23.495 28.575) (width 1.5) (layer "B.Cu") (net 9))
 (segment (start 23.495 28.575) (end 22.225 29.845) (width 1.5) (layer "B.Cu") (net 9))
 (segment (start 64.824999 48.455001) (end 72.970001 48.455001) (width 1.5) (layer "B.Cu") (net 4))
 (segment (start 73.66 47.765002) (end 73.66 46.355) (width 1.5) (layer "B.Cu") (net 4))
 (segment (start 64.135 46.355) (end 64.135 47.765002) (width 1.5) (layer "B.Cu") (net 4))
 (segment (start 64.135 47.765002) (end 64.824999 48.455001) (width 1.5) (layer "B.Cu") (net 4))
 (segment (start 72.970001 48.455001) (end 73.66 47.765002) (width 1.5) (layer "B.Cu") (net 4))
 (segment (start 66.675 46.355) (end 71.12 46.355) (width 1.5) (layer "B.Cu") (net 3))
 (segment (start 59.055 40.64) (end 53.975 35.56) (width 1.5) (layer "B.Cu") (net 21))
 (segment (start 53.975 35.56) (end 53.34 35.56) (width 1.5) (layer "B.Cu") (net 21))
 (segment (start 54.61 33.02) (end 59.055 37.465) (width 1.5) (layer "B.Cu") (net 22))
 (segment (start 53.34 33.02) (end 54.61 33.02) (width 1.5) (layer "B.Cu") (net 22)))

